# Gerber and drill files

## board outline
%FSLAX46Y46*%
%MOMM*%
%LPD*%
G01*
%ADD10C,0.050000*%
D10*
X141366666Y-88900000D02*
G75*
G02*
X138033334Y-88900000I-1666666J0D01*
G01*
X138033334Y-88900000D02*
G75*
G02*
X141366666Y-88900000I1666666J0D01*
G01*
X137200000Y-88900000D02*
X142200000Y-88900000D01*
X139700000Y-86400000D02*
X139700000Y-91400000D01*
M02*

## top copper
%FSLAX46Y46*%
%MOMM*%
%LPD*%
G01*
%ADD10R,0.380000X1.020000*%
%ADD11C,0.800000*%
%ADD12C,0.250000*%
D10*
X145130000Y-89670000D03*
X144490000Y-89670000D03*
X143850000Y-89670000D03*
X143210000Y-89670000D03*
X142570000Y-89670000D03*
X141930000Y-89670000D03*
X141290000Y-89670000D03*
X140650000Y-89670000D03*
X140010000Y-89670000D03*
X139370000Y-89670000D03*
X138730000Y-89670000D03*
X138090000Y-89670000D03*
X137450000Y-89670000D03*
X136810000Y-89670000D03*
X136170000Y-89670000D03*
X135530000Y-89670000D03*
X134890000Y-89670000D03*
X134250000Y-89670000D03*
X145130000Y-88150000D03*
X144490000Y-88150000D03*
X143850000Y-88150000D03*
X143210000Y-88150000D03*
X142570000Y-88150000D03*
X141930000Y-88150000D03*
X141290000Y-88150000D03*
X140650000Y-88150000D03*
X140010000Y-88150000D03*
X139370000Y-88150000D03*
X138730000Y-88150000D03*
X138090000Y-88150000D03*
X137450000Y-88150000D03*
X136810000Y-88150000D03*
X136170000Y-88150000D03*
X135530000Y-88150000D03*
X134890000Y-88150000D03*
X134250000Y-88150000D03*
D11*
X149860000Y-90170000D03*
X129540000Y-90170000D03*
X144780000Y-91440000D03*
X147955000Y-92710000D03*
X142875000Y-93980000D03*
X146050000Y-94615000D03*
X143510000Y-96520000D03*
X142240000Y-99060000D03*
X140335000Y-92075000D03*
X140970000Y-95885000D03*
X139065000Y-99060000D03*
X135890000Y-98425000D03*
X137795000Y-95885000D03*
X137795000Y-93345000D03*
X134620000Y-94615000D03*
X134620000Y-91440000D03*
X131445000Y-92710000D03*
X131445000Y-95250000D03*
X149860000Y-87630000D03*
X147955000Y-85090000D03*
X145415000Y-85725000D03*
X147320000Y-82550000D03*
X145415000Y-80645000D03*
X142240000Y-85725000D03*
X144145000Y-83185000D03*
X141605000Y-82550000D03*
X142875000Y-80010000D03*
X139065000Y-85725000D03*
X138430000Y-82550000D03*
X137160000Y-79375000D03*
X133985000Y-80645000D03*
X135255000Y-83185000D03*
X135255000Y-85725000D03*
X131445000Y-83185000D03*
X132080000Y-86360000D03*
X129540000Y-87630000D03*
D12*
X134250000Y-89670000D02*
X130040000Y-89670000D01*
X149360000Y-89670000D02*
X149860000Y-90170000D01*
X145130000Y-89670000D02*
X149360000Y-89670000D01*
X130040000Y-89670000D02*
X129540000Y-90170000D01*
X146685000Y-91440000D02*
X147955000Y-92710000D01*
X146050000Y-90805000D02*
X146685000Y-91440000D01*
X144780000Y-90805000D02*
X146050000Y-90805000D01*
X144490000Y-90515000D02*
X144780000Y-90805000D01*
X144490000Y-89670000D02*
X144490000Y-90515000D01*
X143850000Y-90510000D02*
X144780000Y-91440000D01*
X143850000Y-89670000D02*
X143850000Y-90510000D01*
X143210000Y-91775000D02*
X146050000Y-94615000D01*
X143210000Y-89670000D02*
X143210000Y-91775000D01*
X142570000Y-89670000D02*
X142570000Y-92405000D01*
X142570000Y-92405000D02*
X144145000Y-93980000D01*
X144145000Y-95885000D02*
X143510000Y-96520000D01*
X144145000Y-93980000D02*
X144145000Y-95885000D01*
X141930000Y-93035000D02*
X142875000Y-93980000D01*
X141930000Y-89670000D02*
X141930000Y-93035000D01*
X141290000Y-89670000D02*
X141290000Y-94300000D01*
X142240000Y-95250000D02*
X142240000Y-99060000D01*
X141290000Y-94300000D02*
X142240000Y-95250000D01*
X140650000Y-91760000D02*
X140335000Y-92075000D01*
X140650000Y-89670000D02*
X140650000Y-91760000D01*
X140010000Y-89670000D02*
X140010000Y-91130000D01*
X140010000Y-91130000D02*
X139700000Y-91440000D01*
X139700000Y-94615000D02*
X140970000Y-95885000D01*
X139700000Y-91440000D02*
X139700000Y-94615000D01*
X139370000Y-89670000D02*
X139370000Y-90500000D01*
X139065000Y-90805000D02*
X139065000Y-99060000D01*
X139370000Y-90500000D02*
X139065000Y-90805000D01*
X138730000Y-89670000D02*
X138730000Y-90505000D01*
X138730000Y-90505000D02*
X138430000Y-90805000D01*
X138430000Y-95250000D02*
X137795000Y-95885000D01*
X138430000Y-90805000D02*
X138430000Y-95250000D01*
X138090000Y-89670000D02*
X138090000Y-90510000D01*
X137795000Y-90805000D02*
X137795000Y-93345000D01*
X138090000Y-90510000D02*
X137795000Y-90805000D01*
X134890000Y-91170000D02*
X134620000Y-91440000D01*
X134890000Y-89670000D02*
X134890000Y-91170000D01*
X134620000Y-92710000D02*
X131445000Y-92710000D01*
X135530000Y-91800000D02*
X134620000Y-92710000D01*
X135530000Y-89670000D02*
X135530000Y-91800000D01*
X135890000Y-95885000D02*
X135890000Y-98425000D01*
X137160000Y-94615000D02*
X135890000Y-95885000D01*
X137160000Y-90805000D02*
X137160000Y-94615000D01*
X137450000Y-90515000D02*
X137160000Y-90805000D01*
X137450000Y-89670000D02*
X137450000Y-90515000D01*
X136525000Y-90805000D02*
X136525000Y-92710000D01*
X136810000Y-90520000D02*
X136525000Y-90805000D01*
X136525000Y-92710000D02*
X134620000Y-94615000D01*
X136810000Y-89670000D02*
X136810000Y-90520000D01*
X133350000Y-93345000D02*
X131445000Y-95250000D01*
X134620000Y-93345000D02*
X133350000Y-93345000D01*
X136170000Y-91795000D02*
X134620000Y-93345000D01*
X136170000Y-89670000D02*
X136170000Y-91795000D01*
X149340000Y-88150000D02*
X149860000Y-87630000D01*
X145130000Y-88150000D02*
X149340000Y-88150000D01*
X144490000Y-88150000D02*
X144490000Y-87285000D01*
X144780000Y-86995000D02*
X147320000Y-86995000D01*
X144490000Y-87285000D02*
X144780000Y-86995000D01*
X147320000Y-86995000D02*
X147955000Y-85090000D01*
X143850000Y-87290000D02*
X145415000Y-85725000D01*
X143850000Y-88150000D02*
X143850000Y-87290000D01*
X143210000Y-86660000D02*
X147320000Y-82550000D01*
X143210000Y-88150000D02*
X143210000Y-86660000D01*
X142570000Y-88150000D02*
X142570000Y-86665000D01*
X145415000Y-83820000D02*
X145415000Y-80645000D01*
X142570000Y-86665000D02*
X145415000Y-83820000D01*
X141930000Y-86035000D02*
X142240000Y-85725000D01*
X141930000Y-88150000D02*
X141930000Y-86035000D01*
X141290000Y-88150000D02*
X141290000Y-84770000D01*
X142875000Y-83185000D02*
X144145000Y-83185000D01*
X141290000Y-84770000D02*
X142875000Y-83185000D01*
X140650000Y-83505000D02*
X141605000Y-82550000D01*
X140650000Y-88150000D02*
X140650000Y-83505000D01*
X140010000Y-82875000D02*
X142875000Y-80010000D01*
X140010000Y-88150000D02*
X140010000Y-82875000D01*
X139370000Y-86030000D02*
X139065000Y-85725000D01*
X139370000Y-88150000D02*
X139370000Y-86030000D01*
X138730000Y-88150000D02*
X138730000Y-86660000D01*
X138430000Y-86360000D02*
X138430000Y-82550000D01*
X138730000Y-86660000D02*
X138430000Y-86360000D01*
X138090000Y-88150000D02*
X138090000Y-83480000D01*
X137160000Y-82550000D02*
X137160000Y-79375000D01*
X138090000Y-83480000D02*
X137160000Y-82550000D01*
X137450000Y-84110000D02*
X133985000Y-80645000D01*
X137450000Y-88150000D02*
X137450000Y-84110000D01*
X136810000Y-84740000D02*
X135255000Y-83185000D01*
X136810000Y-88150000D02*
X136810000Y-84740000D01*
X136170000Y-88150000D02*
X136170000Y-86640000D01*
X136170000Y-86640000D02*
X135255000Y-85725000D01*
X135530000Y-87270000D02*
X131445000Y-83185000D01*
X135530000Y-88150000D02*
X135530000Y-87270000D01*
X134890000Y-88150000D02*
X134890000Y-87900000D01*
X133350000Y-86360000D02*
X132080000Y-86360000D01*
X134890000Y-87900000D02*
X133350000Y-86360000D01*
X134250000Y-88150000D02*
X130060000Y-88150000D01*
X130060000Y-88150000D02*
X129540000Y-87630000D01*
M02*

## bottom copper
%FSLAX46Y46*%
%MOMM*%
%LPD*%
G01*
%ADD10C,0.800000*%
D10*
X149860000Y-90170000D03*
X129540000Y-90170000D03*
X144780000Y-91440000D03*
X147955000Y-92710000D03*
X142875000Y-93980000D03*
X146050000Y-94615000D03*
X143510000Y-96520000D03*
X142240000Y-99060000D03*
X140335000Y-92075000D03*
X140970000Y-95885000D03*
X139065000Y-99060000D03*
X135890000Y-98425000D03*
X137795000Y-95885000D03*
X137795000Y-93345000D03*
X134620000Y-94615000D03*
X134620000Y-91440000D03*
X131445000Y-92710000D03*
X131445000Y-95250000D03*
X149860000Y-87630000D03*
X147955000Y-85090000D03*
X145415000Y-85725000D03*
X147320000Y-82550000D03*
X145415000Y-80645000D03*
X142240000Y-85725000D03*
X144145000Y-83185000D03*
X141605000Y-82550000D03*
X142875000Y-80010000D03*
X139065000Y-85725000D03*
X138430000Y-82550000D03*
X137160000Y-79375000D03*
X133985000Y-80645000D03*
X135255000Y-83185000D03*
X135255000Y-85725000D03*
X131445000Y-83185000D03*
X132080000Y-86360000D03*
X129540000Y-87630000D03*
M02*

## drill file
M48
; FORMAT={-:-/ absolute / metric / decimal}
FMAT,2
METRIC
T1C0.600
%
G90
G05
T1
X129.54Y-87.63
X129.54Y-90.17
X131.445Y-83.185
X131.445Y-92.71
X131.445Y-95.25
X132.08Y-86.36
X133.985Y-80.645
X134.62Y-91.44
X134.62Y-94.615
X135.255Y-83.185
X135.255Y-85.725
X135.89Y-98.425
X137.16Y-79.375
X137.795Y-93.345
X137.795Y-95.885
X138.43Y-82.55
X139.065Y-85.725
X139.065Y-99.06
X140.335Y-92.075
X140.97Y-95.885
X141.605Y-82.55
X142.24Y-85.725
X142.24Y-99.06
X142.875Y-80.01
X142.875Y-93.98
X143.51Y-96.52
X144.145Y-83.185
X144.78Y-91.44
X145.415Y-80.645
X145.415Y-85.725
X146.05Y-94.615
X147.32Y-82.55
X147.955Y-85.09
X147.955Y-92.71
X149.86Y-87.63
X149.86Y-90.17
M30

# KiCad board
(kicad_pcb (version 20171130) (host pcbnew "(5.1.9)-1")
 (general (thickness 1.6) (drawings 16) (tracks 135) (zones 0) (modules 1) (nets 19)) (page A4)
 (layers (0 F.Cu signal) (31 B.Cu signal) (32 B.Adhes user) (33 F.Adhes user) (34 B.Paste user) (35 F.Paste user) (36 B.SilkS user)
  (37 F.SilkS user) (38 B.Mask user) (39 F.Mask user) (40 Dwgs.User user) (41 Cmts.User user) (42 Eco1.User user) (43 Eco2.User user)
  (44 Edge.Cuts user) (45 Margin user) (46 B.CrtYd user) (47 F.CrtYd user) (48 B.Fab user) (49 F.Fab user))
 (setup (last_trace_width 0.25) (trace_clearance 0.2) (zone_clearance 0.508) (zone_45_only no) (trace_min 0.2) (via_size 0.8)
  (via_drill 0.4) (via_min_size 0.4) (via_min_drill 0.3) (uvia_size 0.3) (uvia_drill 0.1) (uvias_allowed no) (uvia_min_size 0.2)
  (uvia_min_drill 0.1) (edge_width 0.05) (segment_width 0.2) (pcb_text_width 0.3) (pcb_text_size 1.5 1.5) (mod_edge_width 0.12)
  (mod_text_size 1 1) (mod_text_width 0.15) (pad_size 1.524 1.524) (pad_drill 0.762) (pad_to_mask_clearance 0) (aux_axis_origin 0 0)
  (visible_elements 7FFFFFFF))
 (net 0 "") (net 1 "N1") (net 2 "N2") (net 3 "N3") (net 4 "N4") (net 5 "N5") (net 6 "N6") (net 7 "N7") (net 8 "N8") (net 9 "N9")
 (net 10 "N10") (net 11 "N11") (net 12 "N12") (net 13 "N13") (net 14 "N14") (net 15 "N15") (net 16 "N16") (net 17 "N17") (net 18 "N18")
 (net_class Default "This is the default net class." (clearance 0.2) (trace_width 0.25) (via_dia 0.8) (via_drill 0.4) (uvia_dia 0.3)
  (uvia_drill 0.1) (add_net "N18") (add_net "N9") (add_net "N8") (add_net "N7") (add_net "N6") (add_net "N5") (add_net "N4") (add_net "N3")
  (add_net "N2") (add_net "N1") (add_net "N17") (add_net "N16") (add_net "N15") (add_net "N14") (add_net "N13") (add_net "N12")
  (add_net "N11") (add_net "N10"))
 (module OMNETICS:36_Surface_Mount (layer F.Cu) (at 139.7 88.9)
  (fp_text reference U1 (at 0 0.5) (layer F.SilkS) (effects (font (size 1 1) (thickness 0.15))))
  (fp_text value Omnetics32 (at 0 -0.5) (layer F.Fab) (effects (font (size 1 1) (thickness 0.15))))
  (pad 36 smd rect (at 5.43 0.77) (size 0.38 1.02) (layers F.Cu F.Paste F.Mask))
  (pad 35 smd rect (at 4.79 0.77) (size 0.38 1.02) (layers F.Cu F.Paste F.Mask))
  (pad 34 smd rect (at 4.15 0.77) (size 0.38 1.02) (layers F.Cu F.Paste F.Mask))
  (pad 33 smd rect (at 3.51 0.77) (size 0.38 1.02) (layers F.Cu F.Paste F.Mask))
  (pad 32 smd rect (at 2.87 0.77) (size 0.38 1.02) (layers F.Cu F.Paste F.Mask))
  (pad 31 smd rect (at 2.23 0.77) (size 0.38 1.02) (layers F.Cu F.Paste F.Mask))
  (pad 30 smd rect (at 1.59 0.77) (size 0.38 1.02) (layers F.Cu F.Paste F.Mask))
  (pad 29 smd rect (at 0.95 0.77) (size 0.38 1.02) (layers F.Cu F.Paste F.Mask))
  (pad 28 smd rect (at 0.31 0.77) (size 0.38 1.02) (layers F.Cu F.Paste F.Mask))
  (pad 27 smd rect (at -0.33 0.77) (size 0.38 1.02) (layers F.Cu F.Paste F.Mask))
  (pad 26 smd rect (at -0.97 0.77) (size 0.38 1.02) (layers F.Cu F.Paste F.Mask))
  (pad 25 smd rect (at -1.61 0.77) (size 0.38 1.02) (layers F.Cu F.Paste F.Mask))
  (pad 24 smd rect (at -2.25 0.77) (size 0.38 1.02) (layers F.Cu F.Paste F.Mask))
  (pad 23 smd rect (at -2.89 0.77) (size 0.38 1.02) (layers F.Cu F.Paste F.Mask))
  (pad 22 smd rect (at -3.53 0.77) (size 0.38 1.02) (layers F.Cu F.Paste F.Mask))
  (pad 21 smd rect (at -4.17 0.77) (size 0.38 1.02) (layers F.Cu F.Paste F.Mask))
  (pad 20 smd rect (at -4.81 0.77) (size 0.38 1.02) (layers F.Cu F.Paste F.Mask))
  (pad 19 smd rect (at -5.45 0.77) (size 0.38 1.02) (layers F.Cu F.Paste F.Mask))
  (pad 18 smd rect (at 5.43 -0.75) (size 0.38 1.02) (layers F.Cu F.Paste F.Mask) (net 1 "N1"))
  (pad 17 smd rect (at 4.79 -0.75) (size 0.38 1.02) (layers F.Cu F.Paste F.Mask) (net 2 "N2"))
  (pad 16 smd rect (at 4.15 -0.75) (size 0.38 1.02) (layers F.Cu F.Paste F.Mask) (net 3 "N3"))
  (pad 15 smd rect (at 3.51 -0.75) (size 0.38 1.02) (layers F.Cu F.Paste F.Mask) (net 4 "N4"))
  (pad 14 smd rect (at 2.87 -0.75) (size 0.38 1.02) (layers F.Cu F.Paste F.Mask) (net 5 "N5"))
  (pad 13 smd rect (at 2.23 -0.75) (size 0.38 1.02) (layers F.Cu F.Paste F.Mask) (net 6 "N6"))
  (pad 12 smd rect (at 1.59 -0.75) (size 0.38 1.02) (layers F.Cu F.Paste F.Mask) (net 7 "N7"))
  (pad 11 smd rect (at 0.95 -0.75) (size 0.38 1.02) (layers F.Cu F.Paste F.Mask) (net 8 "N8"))
  (pad 10 smd rect (at 0.31 -0.75) (size 0.38 1.02) (layers F.Cu F.Paste F.Mask) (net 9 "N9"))
  (pad 9 smd rect (at -0.33 -0.75) (size 0.38 1.02) (layers F.Cu F.Paste F.Mask) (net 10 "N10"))
  (pad 8 smd rect (at -0.97 -0.75) (size 0.38 1.02) (layers F.Cu F.Paste F.Mask) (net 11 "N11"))
  (pad 7 smd rect (at -1.61 -0.75) (size 0.38 1.02) (layers F.Cu F.Paste F.Mask) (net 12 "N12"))
  (pad 6 smd rect (at -2.25 -0.75) (size 0.38 1.02) (layers F.Cu F.Paste F.Mask) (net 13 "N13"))
  (pad 5 smd rect (at -2.89 -0.75) (size 0.38 1.02) (layers F.Cu F.Paste F.Mask) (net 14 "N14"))
  (pad 4 smd rect (at -3.53 -0.75) (size 0.38 1.02) (layers F.Cu F.Paste F.Mask) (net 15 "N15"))
  (pad 3 smd rect (at -4.17 -0.75) (size 0.38 1.02) (layers F.Cu F.Paste F.Mask) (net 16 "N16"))
  (pad 2 smd rect (at -4.81 -0.75) (size 0.38 1.02) (layers F.Cu F.Paste F.Mask) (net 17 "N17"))
  (pad 1 smd rect (at -5.45 -0.75) (size 0.38 1.02) (layers F.Cu F.Paste F.Mask) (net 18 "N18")))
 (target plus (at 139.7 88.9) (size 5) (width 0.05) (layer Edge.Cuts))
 (segment (start 134.25 89.67) (end 130.04 89.67) (width 0.25) (layer F.Cu) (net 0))
 (segment (start 149.36 89.67) (end 149.86 90.17) (width 0.25) (layer F.Cu) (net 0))
 (segment (start 145.13 89.67) (end 149.36 89.67) (width 0.25) (layer F.Cu) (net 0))
 (via (at 149.86 90.17) (size 0.8) (drill 0.6) (layers F.Cu B.Cu) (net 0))
 (segment (start 130.04 89.67) (end 129.54 90.17) (width 0.25) (layer F.Cu) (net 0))
 (via (at 129.54 90.17) (size 0.8) (drill 0.6) (layers F.Cu B.Cu) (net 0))
 (via (at 144.78 91.44) (size 0.8) (drill 0.6) (layers F.Cu B.Cu) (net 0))
 (via (at 147.955 92.71) (size 0.8) (drill 0.6) (layers F.Cu B.Cu) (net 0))
 (via (at 142.875 93.98) (size 0.8) (drill 0.6) (layers F.Cu B.Cu) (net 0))
 (via (at 146.05 94.615) (size 0.8) (drill 0.6) (layers F.Cu B.Cu) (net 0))
 (via (at 143.51 96.52) (size 0.8) (drill 0.6) (layers F.Cu B.Cu) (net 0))
 (via (at 142.24 99.06) (size 0.8) (drill 0.6) (layers F.Cu B.Cu) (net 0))
 (via (at 140.335 92.075) (size 0.8) (drill 0.6) (layers F.Cu B.Cu) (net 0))
 (via (at 140.97 95.885) (size 0.8) (drill 0.6) (layers F.Cu B.Cu) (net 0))
 (via (at 139.065 99.06) (size 0.8) (drill 0.6) (layers F.Cu B.Cu) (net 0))
 (via (at 135.89 98.425) (size 0.8) (drill 0.6) (layers F.Cu B.Cu) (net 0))
 (via (at 137.795 95.885) (size 0.8) (drill 0.6) (layers F.Cu B.Cu) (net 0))
 (via (at 137.795 93.345) (size 0.8) (drill 0.6) (layers F.Cu B.Cu) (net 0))
 (via (at 134.62 94.615) (size 0.8) (drill 0.6) (layers F.Cu B.Cu) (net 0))
 (via (at 134.62 91.44) (size 0.8) (drill 0.6) (layers F.Cu B.Cu) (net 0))
 (via (at 131.445 92.71) (size 0.8) (drill 0.6) (layers F.Cu B.Cu) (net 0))
 (via (at 131.445 95.25) (size 0.8) (drill 0.6) (layers F.Cu B.Cu) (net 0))
 (segment (start 146.685 91.44) (end 147.955 92.71) (width 0.25) (layer F.Cu) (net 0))
 (segment (start 146.05 90.805) (end 146.685 91.44) (width 0.25) (layer F.Cu) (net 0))
 (segment (start 144.78 90.805) (end 146.05 90.805) (width 0.25) (layer F.Cu) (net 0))
 (segment (start 144.49 90.515) (end 144.78 90.805) (width 0.25) (layer F.Cu) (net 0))
 (segment (start 144.49 89.67) (end 144.49 90.515) (width 0.25) (layer F.Cu) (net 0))
 (segment (start 143.85 90.51) (end 144.78 91.44) (width 0.25) (layer F.Cu) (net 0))
 (segment (start 143.85 89.67) (end 143.85 90.51) (width 0.25) (layer F.Cu) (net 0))
 (segment (start 143.21 91.775) (end 146.05 94.615) (width 0.25) (layer F.Cu) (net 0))
 (segment (start 143.21 89.67) (end 143.21 91.775) (width 0.25) (layer F.Cu) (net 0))
 (segment (start 142.57 89.67) (end 142.57 92.405) (width 0.25) (layer F.Cu) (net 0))
 (segment (start 142.57 92.405) (end 144.145 93.98) (width 0.25) (layer F.Cu) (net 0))
 (segment (start 144.145 95.885) (end 143.51 96.52) (width 0.25) (layer F.Cu) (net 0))
 (segment (start 144.145 93.98) (end 144.145 95.885) (width 0.25) (layer F.Cu) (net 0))
 (segment (start 141.93 93.035) (end 142.875 93.98) (width 0.25) (layer F.Cu) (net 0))
 (segment (start 141.93 89.67) (end 141.93 93.035) (width 0.25) (layer F.Cu) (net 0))
 (segment (start 141.29 89.67) (end 141.29 94.3) (width 0.25) (layer F.Cu) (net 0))
 (segment (start 142.24 95.25) (end 142.24 99.06) (width 0.25) (layer F.Cu) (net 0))
 (segment (start 141.29 94.3) (end 142.24 95.25) (width 0.25) (layer F.Cu) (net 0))
 (segment (start 140.65 91.76) (end 140.335 92.075) (width 0.25) (layer F.Cu) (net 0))
 (segment (start 140.65 89.67) (end 140.65 91.76) (width 0.25) (layer F.Cu) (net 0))
 (segment (start 140.01 89.67) (end 140.01 91.13) (width 0.25) (layer F.Cu) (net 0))
 (segment (start 140.01 91.13) (end 139.7 91.44) (width 0.25) (layer F.Cu) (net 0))
 (segment (start 139.7 94.615) (end 140.97 95.885) (width 0.25) (layer F.Cu) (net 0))
 (segment (start 139.7 91.44) (end 139.7 94.615) (width 0.25) (layer F.Cu) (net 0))
 (segment (start 139.37 89.67) (end 139.37 90.5) (width 0.25) (layer F.Cu) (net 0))
 (segment (start 139.065 90.805) (end 139.065 99.06) (width 0.25) (layer F.Cu) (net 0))
 (segment (start 139.37 90.5) (end 139.065 90.805) (width 0.25) (layer F.Cu) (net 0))
 (segment (start 138.73 89.67) (end 138.73 90.505) (width 0.25) (layer F.Cu) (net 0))
 (segment (start 138.73 90.505) (end 138.43 90.805) (width 0.25) (layer F.Cu) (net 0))
 (segment (start 138.43 95.25) (end 137.795 95.885) (width 0.25) (layer F.Cu) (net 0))
 (segment (start 138.43 90.805) (end 138.43 95.25) (width 0.25) (layer F.Cu) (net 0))
 (segment (start 138.09 89.67) (end 138.09 90.51) (width 0.25) (layer F.Cu) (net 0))
 (segment (start 137.795 90.805) (end 137.795 93.345) (width 0.25) (layer F.Cu) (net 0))
 (segment (start 138.09 90.51) (end 137.795 90.805) (width 0.25) (layer F.Cu) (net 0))
 (segment (start 134.89 91.17) (end 134.62 91.44) (width 0.25) (layer F.Cu) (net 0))
 (segment (start 134.89 89.67) (end 134.89 91.17) (width 0.25) (layer F.Cu) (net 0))
 (segment (start 134.62 92.71) (end 131.445 92.71) (width 0.25) (layer F.Cu) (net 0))
 (segment (start 135.53 91.8) (end 134.62 92.71) (width 0.25) (layer F.Cu) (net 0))
 (segment (start 135.53 89.67) (end 135.53 91.8) (width 0.25) (layer F.Cu) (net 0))
 (segment (start 135.89 95.885) (end 135.89 98.425) (width 0.25) (layer F.Cu) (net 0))
 (segment (start 137.16 94.615) (end 135.89 95.885) (width 0.25) (layer F.Cu) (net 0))
 (segment (start 137.16 90.805) (end 137.16 94.615) (width 0.25) (layer F.Cu) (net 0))
 (segment (start 137.45 90.515) (end 137.16 90.805) (width 0.25) (layer F.Cu) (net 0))
 (segment (start 137.45 89.67) (end 137.45 90.515) (width 0.25) (layer F.Cu) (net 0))
 (segment (start 136.525 90.805) (end 136.525 92.71) (width 0.25) (layer F.Cu) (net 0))
 (segment (start 136.81 90.52) (end 136.525 90.805) (width 0.25) (layer F.Cu) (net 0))
 (segment (start 136.525 92.71) (end 134.62 94.615) (width 0.25) (layer F.Cu) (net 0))
 (segment (start 136.81 89.67) (end 136.81 90.52) (width 0.25) (layer F.Cu) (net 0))
 (segment (start 133.35 93.345) (end 131.445 95.25) (width 0.25) (layer F.Cu) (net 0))
 (segment (start 134.62 93.345) (end 133.35 93.345) (width 0.25) (layer F.Cu) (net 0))
 (segment (start 136.17 91.795) (end 134.62 93.345) (width 0.25) (layer F.Cu) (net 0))
 (segment (start 136.17 89.67) (end 136.17 91.795) (width 0.25) (layer F.Cu) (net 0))
 (segment (start 149.34 88.15) (end 149.86 87.63) (width 0.25) (layer F.Cu) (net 1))
 (segment (start 145.13 88.15) (end 149.34 88.15) (width 0.25) (layer F.Cu) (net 1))
 (via (at 149.86 87.63) (size 0.8) (drill 0.6) (layers F.Cu B.Cu) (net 1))
 (via (at 147.955 85.09) (size 0.8) (drill 0.6) (layers F.Cu B.Cu) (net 2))
 (segment (start 144.49 88.15) (end 144.49 87.285) (width 0.25) (layer F.Cu) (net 2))
 (segment (start 144.78 86.995) (end 147.32 86.995) (width 0.25) (layer F.Cu) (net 2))
 (segment (start 144.49 87.285) (end 144.78 86.995) (width 0.25) (layer F.Cu) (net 2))
 (segment (start 147.32 86.995) (end 147.955 85.09) (width 0.25) (layer F.Cu) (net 2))
 (via (at 145.415 85.725) (size 0.8) (drill 0.6) (layers F.Cu B.Cu) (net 3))
 (segment (start 143.85 87.29) (end 145.415 85.725) (width 0.25) (layer F.Cu) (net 3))
 (segment (start 143.85 88.15) (end 143.85 87.29) (width 0.25) (layer F.Cu) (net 3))
 (via (at 147.32 82.55) (size 0.8) (drill 0.6) (layers F.Cu B.Cu) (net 4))
 (segment (start 143.21 86.66) (end 147.32 82.55) (width 0.25) (layer F.Cu) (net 4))
 (segment (start 143.21 88.15) (end 143.21 86.66) (width 0.25) (layer F.Cu) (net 4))
 (via (at 145.415 80.645) (size 0.8) (drill 0.6) (layers F.Cu B.Cu) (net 5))
 (segment (start 142.57 88.15) (end 142.57 86.665) (width 0.25) (layer F.Cu) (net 5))
 (segment (start 145.415 83.82) (end 145.415 80.645) (width 0.25) (layer F.Cu) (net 5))
 (segment (start 142.57 86.665) (end 145.415 83.82) (width 0.25) (layer F.Cu) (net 5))
 (via (at 142.24 85.725) (size 0.8) (drill 0.6) (layers F.Cu B.Cu) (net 6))
 (segment (start 141.93 86.035) (end 142.24 85.725) (width 0.25) (layer F.Cu) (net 6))
 (segment (start 141.93 88.15) (end 141.93 86.035) (width 0.25) (layer F.Cu) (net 6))
 (via (at 144.145 83.185) (size 0.8) (drill 0.6) (layers F.Cu B.Cu) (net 7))
 (segment (start 141.29 88.15) (end 141.29 84.77) (width 0.25) (layer F.Cu) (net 7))
 (segment (start 142.875 83.185) (end 144.145 83.185) (width 0.25) (layer F.Cu) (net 7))
 (segment (start 141.29 84.77) (end 142.875 83.185) (width 0.25) (layer F.Cu) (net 7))
 (via (at 141.605 82.55) (size 0.8) (drill 0.6) (layers F.Cu B.Cu) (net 8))
 (segment (start 140.65 83.505) (end 141.605 82.55) (width 0.25) (layer F.Cu) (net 8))
 (segment (start 140.65 88.15) (end 140.65 83.505) (width 0.25) (layer F.Cu) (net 8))
 (via (at 142.875 80.01) (size 0.8) (drill 0.6) (layers F.Cu B.Cu) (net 9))
 (segment (start 140.01 82.875) (end 142.875 80.01) (width 0.25) (layer F.Cu) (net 9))
 (segment (start 140.01 88.15) (end 140.01 82.875) (width 0.25) (layer F.Cu) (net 9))
 (via (at 139.065 85.725) (size 0.8) (drill 0.6) (layers F.Cu B.Cu) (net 10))
 (segment (start 139.37 86.03) (end 139.065 85.725) (width 0.25) (layer F.Cu) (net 10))
 (segment (start 139.37 88.15) (end 139.37 86.03) (width 0.25) (layer F.Cu) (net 10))
 (via (at 138.43 82.55) (size 0.8) (drill 0.6) (layers F.Cu B.Cu) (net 11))
 (segment (start 138.73 88.15) (end 138.73 86.66) (width 0.25) (layer F.Cu) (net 11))
 (segment (start 138.43 86.36) (end 138.43 82.55) (width 0.25) (layer F.Cu) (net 11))
 (segment (start 138.73 86.66) (end 138.43 86.36) (width 0.25) (layer F.Cu) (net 11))
 (via (at 137.16 79.375) (size 0.8) (drill 0.6) (layers F.Cu B.Cu) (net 12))
 (segment (start 138.09 88.15) (end 138.09 83.48) (width 0.25) (layer F.Cu) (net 12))
 (segment (start 137.16 82.55) (end 137.16 79.375) (width 0.25) (layer F.Cu) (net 12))
 (segment (start 138.09 83.48) (end 137.16 82.55) (width 0.25) (layer F.Cu) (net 12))
 (via (at 133.985 80.645) (size 0.8) (drill 0.6) (layers F.Cu B.Cu) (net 13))
 (segment (start 137.45 84.11) (end 133.985 80.645) (width 0.25) (layer F.Cu) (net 13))
 (segment (start 137.45 88.15) (end 137.45 84.11) (width 0.25) (layer F.Cu) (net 13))
 (via (at 135.255 83.185) (size 0.8) (drill 0.6) (layers F.Cu B.Cu) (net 14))
 (segment (start 136.81 84.74) (end 135.255 83.185) (width 0.25) (layer F.Cu) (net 14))
 (segment (start 136.81 88.15) (end 136.81 84.74) (width 0.25) (layer F.Cu) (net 14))
 (via (at 135.255 85.725) (size 0.8) (drill 0.6) (layers F.Cu B.Cu) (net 15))
 (segment (start 136.17 88.15) (end 136.17 86.64) (width 0.25) (layer F.Cu) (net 15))
 (segment (start 136.17 86.64) (end 135.255 85.725) (width 0.25) (layer F.Cu) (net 15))
 (via (at 131.445 83.185) (size 0.8) (drill 0.6) (layers F.Cu B.Cu) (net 16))
 (segment (start 135.53 87.27) (end 131.445 83.185) (width 0.25) (layer F.Cu) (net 16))
 (segment (start 135.53 88.15) (end 135.53 87.27) (width 0.25) (layer F.Cu) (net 16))
 (via (at 132.08 86.36) (size 0.8) (drill 0.6) (layers F.Cu B.Cu) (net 17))
 (segment (start 134.89 88.15) (end 134.89 87.9) (width 0.25) (layer F.Cu) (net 17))
 (segment (start 133.35 86.36) (end 132.08 86.36) (width 0.25) (layer F.Cu) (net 17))
 (segment (start 134.89 87.9) (end 133.35 86.36) (width 0.25) (layer F.Cu) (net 17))
 (segment (start 134.25 88.15) (end 130.06 88.15) (width 0.25) (layer F.Cu) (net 18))
 (segment (start 130.06 88.15) (end 129.54 87.63) (width 0.25) (layer F.Cu) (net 18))
 (via (at 129.54 87.63) (size 0.8) (drill 0.6) (layers F.Cu B.Cu) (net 18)))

